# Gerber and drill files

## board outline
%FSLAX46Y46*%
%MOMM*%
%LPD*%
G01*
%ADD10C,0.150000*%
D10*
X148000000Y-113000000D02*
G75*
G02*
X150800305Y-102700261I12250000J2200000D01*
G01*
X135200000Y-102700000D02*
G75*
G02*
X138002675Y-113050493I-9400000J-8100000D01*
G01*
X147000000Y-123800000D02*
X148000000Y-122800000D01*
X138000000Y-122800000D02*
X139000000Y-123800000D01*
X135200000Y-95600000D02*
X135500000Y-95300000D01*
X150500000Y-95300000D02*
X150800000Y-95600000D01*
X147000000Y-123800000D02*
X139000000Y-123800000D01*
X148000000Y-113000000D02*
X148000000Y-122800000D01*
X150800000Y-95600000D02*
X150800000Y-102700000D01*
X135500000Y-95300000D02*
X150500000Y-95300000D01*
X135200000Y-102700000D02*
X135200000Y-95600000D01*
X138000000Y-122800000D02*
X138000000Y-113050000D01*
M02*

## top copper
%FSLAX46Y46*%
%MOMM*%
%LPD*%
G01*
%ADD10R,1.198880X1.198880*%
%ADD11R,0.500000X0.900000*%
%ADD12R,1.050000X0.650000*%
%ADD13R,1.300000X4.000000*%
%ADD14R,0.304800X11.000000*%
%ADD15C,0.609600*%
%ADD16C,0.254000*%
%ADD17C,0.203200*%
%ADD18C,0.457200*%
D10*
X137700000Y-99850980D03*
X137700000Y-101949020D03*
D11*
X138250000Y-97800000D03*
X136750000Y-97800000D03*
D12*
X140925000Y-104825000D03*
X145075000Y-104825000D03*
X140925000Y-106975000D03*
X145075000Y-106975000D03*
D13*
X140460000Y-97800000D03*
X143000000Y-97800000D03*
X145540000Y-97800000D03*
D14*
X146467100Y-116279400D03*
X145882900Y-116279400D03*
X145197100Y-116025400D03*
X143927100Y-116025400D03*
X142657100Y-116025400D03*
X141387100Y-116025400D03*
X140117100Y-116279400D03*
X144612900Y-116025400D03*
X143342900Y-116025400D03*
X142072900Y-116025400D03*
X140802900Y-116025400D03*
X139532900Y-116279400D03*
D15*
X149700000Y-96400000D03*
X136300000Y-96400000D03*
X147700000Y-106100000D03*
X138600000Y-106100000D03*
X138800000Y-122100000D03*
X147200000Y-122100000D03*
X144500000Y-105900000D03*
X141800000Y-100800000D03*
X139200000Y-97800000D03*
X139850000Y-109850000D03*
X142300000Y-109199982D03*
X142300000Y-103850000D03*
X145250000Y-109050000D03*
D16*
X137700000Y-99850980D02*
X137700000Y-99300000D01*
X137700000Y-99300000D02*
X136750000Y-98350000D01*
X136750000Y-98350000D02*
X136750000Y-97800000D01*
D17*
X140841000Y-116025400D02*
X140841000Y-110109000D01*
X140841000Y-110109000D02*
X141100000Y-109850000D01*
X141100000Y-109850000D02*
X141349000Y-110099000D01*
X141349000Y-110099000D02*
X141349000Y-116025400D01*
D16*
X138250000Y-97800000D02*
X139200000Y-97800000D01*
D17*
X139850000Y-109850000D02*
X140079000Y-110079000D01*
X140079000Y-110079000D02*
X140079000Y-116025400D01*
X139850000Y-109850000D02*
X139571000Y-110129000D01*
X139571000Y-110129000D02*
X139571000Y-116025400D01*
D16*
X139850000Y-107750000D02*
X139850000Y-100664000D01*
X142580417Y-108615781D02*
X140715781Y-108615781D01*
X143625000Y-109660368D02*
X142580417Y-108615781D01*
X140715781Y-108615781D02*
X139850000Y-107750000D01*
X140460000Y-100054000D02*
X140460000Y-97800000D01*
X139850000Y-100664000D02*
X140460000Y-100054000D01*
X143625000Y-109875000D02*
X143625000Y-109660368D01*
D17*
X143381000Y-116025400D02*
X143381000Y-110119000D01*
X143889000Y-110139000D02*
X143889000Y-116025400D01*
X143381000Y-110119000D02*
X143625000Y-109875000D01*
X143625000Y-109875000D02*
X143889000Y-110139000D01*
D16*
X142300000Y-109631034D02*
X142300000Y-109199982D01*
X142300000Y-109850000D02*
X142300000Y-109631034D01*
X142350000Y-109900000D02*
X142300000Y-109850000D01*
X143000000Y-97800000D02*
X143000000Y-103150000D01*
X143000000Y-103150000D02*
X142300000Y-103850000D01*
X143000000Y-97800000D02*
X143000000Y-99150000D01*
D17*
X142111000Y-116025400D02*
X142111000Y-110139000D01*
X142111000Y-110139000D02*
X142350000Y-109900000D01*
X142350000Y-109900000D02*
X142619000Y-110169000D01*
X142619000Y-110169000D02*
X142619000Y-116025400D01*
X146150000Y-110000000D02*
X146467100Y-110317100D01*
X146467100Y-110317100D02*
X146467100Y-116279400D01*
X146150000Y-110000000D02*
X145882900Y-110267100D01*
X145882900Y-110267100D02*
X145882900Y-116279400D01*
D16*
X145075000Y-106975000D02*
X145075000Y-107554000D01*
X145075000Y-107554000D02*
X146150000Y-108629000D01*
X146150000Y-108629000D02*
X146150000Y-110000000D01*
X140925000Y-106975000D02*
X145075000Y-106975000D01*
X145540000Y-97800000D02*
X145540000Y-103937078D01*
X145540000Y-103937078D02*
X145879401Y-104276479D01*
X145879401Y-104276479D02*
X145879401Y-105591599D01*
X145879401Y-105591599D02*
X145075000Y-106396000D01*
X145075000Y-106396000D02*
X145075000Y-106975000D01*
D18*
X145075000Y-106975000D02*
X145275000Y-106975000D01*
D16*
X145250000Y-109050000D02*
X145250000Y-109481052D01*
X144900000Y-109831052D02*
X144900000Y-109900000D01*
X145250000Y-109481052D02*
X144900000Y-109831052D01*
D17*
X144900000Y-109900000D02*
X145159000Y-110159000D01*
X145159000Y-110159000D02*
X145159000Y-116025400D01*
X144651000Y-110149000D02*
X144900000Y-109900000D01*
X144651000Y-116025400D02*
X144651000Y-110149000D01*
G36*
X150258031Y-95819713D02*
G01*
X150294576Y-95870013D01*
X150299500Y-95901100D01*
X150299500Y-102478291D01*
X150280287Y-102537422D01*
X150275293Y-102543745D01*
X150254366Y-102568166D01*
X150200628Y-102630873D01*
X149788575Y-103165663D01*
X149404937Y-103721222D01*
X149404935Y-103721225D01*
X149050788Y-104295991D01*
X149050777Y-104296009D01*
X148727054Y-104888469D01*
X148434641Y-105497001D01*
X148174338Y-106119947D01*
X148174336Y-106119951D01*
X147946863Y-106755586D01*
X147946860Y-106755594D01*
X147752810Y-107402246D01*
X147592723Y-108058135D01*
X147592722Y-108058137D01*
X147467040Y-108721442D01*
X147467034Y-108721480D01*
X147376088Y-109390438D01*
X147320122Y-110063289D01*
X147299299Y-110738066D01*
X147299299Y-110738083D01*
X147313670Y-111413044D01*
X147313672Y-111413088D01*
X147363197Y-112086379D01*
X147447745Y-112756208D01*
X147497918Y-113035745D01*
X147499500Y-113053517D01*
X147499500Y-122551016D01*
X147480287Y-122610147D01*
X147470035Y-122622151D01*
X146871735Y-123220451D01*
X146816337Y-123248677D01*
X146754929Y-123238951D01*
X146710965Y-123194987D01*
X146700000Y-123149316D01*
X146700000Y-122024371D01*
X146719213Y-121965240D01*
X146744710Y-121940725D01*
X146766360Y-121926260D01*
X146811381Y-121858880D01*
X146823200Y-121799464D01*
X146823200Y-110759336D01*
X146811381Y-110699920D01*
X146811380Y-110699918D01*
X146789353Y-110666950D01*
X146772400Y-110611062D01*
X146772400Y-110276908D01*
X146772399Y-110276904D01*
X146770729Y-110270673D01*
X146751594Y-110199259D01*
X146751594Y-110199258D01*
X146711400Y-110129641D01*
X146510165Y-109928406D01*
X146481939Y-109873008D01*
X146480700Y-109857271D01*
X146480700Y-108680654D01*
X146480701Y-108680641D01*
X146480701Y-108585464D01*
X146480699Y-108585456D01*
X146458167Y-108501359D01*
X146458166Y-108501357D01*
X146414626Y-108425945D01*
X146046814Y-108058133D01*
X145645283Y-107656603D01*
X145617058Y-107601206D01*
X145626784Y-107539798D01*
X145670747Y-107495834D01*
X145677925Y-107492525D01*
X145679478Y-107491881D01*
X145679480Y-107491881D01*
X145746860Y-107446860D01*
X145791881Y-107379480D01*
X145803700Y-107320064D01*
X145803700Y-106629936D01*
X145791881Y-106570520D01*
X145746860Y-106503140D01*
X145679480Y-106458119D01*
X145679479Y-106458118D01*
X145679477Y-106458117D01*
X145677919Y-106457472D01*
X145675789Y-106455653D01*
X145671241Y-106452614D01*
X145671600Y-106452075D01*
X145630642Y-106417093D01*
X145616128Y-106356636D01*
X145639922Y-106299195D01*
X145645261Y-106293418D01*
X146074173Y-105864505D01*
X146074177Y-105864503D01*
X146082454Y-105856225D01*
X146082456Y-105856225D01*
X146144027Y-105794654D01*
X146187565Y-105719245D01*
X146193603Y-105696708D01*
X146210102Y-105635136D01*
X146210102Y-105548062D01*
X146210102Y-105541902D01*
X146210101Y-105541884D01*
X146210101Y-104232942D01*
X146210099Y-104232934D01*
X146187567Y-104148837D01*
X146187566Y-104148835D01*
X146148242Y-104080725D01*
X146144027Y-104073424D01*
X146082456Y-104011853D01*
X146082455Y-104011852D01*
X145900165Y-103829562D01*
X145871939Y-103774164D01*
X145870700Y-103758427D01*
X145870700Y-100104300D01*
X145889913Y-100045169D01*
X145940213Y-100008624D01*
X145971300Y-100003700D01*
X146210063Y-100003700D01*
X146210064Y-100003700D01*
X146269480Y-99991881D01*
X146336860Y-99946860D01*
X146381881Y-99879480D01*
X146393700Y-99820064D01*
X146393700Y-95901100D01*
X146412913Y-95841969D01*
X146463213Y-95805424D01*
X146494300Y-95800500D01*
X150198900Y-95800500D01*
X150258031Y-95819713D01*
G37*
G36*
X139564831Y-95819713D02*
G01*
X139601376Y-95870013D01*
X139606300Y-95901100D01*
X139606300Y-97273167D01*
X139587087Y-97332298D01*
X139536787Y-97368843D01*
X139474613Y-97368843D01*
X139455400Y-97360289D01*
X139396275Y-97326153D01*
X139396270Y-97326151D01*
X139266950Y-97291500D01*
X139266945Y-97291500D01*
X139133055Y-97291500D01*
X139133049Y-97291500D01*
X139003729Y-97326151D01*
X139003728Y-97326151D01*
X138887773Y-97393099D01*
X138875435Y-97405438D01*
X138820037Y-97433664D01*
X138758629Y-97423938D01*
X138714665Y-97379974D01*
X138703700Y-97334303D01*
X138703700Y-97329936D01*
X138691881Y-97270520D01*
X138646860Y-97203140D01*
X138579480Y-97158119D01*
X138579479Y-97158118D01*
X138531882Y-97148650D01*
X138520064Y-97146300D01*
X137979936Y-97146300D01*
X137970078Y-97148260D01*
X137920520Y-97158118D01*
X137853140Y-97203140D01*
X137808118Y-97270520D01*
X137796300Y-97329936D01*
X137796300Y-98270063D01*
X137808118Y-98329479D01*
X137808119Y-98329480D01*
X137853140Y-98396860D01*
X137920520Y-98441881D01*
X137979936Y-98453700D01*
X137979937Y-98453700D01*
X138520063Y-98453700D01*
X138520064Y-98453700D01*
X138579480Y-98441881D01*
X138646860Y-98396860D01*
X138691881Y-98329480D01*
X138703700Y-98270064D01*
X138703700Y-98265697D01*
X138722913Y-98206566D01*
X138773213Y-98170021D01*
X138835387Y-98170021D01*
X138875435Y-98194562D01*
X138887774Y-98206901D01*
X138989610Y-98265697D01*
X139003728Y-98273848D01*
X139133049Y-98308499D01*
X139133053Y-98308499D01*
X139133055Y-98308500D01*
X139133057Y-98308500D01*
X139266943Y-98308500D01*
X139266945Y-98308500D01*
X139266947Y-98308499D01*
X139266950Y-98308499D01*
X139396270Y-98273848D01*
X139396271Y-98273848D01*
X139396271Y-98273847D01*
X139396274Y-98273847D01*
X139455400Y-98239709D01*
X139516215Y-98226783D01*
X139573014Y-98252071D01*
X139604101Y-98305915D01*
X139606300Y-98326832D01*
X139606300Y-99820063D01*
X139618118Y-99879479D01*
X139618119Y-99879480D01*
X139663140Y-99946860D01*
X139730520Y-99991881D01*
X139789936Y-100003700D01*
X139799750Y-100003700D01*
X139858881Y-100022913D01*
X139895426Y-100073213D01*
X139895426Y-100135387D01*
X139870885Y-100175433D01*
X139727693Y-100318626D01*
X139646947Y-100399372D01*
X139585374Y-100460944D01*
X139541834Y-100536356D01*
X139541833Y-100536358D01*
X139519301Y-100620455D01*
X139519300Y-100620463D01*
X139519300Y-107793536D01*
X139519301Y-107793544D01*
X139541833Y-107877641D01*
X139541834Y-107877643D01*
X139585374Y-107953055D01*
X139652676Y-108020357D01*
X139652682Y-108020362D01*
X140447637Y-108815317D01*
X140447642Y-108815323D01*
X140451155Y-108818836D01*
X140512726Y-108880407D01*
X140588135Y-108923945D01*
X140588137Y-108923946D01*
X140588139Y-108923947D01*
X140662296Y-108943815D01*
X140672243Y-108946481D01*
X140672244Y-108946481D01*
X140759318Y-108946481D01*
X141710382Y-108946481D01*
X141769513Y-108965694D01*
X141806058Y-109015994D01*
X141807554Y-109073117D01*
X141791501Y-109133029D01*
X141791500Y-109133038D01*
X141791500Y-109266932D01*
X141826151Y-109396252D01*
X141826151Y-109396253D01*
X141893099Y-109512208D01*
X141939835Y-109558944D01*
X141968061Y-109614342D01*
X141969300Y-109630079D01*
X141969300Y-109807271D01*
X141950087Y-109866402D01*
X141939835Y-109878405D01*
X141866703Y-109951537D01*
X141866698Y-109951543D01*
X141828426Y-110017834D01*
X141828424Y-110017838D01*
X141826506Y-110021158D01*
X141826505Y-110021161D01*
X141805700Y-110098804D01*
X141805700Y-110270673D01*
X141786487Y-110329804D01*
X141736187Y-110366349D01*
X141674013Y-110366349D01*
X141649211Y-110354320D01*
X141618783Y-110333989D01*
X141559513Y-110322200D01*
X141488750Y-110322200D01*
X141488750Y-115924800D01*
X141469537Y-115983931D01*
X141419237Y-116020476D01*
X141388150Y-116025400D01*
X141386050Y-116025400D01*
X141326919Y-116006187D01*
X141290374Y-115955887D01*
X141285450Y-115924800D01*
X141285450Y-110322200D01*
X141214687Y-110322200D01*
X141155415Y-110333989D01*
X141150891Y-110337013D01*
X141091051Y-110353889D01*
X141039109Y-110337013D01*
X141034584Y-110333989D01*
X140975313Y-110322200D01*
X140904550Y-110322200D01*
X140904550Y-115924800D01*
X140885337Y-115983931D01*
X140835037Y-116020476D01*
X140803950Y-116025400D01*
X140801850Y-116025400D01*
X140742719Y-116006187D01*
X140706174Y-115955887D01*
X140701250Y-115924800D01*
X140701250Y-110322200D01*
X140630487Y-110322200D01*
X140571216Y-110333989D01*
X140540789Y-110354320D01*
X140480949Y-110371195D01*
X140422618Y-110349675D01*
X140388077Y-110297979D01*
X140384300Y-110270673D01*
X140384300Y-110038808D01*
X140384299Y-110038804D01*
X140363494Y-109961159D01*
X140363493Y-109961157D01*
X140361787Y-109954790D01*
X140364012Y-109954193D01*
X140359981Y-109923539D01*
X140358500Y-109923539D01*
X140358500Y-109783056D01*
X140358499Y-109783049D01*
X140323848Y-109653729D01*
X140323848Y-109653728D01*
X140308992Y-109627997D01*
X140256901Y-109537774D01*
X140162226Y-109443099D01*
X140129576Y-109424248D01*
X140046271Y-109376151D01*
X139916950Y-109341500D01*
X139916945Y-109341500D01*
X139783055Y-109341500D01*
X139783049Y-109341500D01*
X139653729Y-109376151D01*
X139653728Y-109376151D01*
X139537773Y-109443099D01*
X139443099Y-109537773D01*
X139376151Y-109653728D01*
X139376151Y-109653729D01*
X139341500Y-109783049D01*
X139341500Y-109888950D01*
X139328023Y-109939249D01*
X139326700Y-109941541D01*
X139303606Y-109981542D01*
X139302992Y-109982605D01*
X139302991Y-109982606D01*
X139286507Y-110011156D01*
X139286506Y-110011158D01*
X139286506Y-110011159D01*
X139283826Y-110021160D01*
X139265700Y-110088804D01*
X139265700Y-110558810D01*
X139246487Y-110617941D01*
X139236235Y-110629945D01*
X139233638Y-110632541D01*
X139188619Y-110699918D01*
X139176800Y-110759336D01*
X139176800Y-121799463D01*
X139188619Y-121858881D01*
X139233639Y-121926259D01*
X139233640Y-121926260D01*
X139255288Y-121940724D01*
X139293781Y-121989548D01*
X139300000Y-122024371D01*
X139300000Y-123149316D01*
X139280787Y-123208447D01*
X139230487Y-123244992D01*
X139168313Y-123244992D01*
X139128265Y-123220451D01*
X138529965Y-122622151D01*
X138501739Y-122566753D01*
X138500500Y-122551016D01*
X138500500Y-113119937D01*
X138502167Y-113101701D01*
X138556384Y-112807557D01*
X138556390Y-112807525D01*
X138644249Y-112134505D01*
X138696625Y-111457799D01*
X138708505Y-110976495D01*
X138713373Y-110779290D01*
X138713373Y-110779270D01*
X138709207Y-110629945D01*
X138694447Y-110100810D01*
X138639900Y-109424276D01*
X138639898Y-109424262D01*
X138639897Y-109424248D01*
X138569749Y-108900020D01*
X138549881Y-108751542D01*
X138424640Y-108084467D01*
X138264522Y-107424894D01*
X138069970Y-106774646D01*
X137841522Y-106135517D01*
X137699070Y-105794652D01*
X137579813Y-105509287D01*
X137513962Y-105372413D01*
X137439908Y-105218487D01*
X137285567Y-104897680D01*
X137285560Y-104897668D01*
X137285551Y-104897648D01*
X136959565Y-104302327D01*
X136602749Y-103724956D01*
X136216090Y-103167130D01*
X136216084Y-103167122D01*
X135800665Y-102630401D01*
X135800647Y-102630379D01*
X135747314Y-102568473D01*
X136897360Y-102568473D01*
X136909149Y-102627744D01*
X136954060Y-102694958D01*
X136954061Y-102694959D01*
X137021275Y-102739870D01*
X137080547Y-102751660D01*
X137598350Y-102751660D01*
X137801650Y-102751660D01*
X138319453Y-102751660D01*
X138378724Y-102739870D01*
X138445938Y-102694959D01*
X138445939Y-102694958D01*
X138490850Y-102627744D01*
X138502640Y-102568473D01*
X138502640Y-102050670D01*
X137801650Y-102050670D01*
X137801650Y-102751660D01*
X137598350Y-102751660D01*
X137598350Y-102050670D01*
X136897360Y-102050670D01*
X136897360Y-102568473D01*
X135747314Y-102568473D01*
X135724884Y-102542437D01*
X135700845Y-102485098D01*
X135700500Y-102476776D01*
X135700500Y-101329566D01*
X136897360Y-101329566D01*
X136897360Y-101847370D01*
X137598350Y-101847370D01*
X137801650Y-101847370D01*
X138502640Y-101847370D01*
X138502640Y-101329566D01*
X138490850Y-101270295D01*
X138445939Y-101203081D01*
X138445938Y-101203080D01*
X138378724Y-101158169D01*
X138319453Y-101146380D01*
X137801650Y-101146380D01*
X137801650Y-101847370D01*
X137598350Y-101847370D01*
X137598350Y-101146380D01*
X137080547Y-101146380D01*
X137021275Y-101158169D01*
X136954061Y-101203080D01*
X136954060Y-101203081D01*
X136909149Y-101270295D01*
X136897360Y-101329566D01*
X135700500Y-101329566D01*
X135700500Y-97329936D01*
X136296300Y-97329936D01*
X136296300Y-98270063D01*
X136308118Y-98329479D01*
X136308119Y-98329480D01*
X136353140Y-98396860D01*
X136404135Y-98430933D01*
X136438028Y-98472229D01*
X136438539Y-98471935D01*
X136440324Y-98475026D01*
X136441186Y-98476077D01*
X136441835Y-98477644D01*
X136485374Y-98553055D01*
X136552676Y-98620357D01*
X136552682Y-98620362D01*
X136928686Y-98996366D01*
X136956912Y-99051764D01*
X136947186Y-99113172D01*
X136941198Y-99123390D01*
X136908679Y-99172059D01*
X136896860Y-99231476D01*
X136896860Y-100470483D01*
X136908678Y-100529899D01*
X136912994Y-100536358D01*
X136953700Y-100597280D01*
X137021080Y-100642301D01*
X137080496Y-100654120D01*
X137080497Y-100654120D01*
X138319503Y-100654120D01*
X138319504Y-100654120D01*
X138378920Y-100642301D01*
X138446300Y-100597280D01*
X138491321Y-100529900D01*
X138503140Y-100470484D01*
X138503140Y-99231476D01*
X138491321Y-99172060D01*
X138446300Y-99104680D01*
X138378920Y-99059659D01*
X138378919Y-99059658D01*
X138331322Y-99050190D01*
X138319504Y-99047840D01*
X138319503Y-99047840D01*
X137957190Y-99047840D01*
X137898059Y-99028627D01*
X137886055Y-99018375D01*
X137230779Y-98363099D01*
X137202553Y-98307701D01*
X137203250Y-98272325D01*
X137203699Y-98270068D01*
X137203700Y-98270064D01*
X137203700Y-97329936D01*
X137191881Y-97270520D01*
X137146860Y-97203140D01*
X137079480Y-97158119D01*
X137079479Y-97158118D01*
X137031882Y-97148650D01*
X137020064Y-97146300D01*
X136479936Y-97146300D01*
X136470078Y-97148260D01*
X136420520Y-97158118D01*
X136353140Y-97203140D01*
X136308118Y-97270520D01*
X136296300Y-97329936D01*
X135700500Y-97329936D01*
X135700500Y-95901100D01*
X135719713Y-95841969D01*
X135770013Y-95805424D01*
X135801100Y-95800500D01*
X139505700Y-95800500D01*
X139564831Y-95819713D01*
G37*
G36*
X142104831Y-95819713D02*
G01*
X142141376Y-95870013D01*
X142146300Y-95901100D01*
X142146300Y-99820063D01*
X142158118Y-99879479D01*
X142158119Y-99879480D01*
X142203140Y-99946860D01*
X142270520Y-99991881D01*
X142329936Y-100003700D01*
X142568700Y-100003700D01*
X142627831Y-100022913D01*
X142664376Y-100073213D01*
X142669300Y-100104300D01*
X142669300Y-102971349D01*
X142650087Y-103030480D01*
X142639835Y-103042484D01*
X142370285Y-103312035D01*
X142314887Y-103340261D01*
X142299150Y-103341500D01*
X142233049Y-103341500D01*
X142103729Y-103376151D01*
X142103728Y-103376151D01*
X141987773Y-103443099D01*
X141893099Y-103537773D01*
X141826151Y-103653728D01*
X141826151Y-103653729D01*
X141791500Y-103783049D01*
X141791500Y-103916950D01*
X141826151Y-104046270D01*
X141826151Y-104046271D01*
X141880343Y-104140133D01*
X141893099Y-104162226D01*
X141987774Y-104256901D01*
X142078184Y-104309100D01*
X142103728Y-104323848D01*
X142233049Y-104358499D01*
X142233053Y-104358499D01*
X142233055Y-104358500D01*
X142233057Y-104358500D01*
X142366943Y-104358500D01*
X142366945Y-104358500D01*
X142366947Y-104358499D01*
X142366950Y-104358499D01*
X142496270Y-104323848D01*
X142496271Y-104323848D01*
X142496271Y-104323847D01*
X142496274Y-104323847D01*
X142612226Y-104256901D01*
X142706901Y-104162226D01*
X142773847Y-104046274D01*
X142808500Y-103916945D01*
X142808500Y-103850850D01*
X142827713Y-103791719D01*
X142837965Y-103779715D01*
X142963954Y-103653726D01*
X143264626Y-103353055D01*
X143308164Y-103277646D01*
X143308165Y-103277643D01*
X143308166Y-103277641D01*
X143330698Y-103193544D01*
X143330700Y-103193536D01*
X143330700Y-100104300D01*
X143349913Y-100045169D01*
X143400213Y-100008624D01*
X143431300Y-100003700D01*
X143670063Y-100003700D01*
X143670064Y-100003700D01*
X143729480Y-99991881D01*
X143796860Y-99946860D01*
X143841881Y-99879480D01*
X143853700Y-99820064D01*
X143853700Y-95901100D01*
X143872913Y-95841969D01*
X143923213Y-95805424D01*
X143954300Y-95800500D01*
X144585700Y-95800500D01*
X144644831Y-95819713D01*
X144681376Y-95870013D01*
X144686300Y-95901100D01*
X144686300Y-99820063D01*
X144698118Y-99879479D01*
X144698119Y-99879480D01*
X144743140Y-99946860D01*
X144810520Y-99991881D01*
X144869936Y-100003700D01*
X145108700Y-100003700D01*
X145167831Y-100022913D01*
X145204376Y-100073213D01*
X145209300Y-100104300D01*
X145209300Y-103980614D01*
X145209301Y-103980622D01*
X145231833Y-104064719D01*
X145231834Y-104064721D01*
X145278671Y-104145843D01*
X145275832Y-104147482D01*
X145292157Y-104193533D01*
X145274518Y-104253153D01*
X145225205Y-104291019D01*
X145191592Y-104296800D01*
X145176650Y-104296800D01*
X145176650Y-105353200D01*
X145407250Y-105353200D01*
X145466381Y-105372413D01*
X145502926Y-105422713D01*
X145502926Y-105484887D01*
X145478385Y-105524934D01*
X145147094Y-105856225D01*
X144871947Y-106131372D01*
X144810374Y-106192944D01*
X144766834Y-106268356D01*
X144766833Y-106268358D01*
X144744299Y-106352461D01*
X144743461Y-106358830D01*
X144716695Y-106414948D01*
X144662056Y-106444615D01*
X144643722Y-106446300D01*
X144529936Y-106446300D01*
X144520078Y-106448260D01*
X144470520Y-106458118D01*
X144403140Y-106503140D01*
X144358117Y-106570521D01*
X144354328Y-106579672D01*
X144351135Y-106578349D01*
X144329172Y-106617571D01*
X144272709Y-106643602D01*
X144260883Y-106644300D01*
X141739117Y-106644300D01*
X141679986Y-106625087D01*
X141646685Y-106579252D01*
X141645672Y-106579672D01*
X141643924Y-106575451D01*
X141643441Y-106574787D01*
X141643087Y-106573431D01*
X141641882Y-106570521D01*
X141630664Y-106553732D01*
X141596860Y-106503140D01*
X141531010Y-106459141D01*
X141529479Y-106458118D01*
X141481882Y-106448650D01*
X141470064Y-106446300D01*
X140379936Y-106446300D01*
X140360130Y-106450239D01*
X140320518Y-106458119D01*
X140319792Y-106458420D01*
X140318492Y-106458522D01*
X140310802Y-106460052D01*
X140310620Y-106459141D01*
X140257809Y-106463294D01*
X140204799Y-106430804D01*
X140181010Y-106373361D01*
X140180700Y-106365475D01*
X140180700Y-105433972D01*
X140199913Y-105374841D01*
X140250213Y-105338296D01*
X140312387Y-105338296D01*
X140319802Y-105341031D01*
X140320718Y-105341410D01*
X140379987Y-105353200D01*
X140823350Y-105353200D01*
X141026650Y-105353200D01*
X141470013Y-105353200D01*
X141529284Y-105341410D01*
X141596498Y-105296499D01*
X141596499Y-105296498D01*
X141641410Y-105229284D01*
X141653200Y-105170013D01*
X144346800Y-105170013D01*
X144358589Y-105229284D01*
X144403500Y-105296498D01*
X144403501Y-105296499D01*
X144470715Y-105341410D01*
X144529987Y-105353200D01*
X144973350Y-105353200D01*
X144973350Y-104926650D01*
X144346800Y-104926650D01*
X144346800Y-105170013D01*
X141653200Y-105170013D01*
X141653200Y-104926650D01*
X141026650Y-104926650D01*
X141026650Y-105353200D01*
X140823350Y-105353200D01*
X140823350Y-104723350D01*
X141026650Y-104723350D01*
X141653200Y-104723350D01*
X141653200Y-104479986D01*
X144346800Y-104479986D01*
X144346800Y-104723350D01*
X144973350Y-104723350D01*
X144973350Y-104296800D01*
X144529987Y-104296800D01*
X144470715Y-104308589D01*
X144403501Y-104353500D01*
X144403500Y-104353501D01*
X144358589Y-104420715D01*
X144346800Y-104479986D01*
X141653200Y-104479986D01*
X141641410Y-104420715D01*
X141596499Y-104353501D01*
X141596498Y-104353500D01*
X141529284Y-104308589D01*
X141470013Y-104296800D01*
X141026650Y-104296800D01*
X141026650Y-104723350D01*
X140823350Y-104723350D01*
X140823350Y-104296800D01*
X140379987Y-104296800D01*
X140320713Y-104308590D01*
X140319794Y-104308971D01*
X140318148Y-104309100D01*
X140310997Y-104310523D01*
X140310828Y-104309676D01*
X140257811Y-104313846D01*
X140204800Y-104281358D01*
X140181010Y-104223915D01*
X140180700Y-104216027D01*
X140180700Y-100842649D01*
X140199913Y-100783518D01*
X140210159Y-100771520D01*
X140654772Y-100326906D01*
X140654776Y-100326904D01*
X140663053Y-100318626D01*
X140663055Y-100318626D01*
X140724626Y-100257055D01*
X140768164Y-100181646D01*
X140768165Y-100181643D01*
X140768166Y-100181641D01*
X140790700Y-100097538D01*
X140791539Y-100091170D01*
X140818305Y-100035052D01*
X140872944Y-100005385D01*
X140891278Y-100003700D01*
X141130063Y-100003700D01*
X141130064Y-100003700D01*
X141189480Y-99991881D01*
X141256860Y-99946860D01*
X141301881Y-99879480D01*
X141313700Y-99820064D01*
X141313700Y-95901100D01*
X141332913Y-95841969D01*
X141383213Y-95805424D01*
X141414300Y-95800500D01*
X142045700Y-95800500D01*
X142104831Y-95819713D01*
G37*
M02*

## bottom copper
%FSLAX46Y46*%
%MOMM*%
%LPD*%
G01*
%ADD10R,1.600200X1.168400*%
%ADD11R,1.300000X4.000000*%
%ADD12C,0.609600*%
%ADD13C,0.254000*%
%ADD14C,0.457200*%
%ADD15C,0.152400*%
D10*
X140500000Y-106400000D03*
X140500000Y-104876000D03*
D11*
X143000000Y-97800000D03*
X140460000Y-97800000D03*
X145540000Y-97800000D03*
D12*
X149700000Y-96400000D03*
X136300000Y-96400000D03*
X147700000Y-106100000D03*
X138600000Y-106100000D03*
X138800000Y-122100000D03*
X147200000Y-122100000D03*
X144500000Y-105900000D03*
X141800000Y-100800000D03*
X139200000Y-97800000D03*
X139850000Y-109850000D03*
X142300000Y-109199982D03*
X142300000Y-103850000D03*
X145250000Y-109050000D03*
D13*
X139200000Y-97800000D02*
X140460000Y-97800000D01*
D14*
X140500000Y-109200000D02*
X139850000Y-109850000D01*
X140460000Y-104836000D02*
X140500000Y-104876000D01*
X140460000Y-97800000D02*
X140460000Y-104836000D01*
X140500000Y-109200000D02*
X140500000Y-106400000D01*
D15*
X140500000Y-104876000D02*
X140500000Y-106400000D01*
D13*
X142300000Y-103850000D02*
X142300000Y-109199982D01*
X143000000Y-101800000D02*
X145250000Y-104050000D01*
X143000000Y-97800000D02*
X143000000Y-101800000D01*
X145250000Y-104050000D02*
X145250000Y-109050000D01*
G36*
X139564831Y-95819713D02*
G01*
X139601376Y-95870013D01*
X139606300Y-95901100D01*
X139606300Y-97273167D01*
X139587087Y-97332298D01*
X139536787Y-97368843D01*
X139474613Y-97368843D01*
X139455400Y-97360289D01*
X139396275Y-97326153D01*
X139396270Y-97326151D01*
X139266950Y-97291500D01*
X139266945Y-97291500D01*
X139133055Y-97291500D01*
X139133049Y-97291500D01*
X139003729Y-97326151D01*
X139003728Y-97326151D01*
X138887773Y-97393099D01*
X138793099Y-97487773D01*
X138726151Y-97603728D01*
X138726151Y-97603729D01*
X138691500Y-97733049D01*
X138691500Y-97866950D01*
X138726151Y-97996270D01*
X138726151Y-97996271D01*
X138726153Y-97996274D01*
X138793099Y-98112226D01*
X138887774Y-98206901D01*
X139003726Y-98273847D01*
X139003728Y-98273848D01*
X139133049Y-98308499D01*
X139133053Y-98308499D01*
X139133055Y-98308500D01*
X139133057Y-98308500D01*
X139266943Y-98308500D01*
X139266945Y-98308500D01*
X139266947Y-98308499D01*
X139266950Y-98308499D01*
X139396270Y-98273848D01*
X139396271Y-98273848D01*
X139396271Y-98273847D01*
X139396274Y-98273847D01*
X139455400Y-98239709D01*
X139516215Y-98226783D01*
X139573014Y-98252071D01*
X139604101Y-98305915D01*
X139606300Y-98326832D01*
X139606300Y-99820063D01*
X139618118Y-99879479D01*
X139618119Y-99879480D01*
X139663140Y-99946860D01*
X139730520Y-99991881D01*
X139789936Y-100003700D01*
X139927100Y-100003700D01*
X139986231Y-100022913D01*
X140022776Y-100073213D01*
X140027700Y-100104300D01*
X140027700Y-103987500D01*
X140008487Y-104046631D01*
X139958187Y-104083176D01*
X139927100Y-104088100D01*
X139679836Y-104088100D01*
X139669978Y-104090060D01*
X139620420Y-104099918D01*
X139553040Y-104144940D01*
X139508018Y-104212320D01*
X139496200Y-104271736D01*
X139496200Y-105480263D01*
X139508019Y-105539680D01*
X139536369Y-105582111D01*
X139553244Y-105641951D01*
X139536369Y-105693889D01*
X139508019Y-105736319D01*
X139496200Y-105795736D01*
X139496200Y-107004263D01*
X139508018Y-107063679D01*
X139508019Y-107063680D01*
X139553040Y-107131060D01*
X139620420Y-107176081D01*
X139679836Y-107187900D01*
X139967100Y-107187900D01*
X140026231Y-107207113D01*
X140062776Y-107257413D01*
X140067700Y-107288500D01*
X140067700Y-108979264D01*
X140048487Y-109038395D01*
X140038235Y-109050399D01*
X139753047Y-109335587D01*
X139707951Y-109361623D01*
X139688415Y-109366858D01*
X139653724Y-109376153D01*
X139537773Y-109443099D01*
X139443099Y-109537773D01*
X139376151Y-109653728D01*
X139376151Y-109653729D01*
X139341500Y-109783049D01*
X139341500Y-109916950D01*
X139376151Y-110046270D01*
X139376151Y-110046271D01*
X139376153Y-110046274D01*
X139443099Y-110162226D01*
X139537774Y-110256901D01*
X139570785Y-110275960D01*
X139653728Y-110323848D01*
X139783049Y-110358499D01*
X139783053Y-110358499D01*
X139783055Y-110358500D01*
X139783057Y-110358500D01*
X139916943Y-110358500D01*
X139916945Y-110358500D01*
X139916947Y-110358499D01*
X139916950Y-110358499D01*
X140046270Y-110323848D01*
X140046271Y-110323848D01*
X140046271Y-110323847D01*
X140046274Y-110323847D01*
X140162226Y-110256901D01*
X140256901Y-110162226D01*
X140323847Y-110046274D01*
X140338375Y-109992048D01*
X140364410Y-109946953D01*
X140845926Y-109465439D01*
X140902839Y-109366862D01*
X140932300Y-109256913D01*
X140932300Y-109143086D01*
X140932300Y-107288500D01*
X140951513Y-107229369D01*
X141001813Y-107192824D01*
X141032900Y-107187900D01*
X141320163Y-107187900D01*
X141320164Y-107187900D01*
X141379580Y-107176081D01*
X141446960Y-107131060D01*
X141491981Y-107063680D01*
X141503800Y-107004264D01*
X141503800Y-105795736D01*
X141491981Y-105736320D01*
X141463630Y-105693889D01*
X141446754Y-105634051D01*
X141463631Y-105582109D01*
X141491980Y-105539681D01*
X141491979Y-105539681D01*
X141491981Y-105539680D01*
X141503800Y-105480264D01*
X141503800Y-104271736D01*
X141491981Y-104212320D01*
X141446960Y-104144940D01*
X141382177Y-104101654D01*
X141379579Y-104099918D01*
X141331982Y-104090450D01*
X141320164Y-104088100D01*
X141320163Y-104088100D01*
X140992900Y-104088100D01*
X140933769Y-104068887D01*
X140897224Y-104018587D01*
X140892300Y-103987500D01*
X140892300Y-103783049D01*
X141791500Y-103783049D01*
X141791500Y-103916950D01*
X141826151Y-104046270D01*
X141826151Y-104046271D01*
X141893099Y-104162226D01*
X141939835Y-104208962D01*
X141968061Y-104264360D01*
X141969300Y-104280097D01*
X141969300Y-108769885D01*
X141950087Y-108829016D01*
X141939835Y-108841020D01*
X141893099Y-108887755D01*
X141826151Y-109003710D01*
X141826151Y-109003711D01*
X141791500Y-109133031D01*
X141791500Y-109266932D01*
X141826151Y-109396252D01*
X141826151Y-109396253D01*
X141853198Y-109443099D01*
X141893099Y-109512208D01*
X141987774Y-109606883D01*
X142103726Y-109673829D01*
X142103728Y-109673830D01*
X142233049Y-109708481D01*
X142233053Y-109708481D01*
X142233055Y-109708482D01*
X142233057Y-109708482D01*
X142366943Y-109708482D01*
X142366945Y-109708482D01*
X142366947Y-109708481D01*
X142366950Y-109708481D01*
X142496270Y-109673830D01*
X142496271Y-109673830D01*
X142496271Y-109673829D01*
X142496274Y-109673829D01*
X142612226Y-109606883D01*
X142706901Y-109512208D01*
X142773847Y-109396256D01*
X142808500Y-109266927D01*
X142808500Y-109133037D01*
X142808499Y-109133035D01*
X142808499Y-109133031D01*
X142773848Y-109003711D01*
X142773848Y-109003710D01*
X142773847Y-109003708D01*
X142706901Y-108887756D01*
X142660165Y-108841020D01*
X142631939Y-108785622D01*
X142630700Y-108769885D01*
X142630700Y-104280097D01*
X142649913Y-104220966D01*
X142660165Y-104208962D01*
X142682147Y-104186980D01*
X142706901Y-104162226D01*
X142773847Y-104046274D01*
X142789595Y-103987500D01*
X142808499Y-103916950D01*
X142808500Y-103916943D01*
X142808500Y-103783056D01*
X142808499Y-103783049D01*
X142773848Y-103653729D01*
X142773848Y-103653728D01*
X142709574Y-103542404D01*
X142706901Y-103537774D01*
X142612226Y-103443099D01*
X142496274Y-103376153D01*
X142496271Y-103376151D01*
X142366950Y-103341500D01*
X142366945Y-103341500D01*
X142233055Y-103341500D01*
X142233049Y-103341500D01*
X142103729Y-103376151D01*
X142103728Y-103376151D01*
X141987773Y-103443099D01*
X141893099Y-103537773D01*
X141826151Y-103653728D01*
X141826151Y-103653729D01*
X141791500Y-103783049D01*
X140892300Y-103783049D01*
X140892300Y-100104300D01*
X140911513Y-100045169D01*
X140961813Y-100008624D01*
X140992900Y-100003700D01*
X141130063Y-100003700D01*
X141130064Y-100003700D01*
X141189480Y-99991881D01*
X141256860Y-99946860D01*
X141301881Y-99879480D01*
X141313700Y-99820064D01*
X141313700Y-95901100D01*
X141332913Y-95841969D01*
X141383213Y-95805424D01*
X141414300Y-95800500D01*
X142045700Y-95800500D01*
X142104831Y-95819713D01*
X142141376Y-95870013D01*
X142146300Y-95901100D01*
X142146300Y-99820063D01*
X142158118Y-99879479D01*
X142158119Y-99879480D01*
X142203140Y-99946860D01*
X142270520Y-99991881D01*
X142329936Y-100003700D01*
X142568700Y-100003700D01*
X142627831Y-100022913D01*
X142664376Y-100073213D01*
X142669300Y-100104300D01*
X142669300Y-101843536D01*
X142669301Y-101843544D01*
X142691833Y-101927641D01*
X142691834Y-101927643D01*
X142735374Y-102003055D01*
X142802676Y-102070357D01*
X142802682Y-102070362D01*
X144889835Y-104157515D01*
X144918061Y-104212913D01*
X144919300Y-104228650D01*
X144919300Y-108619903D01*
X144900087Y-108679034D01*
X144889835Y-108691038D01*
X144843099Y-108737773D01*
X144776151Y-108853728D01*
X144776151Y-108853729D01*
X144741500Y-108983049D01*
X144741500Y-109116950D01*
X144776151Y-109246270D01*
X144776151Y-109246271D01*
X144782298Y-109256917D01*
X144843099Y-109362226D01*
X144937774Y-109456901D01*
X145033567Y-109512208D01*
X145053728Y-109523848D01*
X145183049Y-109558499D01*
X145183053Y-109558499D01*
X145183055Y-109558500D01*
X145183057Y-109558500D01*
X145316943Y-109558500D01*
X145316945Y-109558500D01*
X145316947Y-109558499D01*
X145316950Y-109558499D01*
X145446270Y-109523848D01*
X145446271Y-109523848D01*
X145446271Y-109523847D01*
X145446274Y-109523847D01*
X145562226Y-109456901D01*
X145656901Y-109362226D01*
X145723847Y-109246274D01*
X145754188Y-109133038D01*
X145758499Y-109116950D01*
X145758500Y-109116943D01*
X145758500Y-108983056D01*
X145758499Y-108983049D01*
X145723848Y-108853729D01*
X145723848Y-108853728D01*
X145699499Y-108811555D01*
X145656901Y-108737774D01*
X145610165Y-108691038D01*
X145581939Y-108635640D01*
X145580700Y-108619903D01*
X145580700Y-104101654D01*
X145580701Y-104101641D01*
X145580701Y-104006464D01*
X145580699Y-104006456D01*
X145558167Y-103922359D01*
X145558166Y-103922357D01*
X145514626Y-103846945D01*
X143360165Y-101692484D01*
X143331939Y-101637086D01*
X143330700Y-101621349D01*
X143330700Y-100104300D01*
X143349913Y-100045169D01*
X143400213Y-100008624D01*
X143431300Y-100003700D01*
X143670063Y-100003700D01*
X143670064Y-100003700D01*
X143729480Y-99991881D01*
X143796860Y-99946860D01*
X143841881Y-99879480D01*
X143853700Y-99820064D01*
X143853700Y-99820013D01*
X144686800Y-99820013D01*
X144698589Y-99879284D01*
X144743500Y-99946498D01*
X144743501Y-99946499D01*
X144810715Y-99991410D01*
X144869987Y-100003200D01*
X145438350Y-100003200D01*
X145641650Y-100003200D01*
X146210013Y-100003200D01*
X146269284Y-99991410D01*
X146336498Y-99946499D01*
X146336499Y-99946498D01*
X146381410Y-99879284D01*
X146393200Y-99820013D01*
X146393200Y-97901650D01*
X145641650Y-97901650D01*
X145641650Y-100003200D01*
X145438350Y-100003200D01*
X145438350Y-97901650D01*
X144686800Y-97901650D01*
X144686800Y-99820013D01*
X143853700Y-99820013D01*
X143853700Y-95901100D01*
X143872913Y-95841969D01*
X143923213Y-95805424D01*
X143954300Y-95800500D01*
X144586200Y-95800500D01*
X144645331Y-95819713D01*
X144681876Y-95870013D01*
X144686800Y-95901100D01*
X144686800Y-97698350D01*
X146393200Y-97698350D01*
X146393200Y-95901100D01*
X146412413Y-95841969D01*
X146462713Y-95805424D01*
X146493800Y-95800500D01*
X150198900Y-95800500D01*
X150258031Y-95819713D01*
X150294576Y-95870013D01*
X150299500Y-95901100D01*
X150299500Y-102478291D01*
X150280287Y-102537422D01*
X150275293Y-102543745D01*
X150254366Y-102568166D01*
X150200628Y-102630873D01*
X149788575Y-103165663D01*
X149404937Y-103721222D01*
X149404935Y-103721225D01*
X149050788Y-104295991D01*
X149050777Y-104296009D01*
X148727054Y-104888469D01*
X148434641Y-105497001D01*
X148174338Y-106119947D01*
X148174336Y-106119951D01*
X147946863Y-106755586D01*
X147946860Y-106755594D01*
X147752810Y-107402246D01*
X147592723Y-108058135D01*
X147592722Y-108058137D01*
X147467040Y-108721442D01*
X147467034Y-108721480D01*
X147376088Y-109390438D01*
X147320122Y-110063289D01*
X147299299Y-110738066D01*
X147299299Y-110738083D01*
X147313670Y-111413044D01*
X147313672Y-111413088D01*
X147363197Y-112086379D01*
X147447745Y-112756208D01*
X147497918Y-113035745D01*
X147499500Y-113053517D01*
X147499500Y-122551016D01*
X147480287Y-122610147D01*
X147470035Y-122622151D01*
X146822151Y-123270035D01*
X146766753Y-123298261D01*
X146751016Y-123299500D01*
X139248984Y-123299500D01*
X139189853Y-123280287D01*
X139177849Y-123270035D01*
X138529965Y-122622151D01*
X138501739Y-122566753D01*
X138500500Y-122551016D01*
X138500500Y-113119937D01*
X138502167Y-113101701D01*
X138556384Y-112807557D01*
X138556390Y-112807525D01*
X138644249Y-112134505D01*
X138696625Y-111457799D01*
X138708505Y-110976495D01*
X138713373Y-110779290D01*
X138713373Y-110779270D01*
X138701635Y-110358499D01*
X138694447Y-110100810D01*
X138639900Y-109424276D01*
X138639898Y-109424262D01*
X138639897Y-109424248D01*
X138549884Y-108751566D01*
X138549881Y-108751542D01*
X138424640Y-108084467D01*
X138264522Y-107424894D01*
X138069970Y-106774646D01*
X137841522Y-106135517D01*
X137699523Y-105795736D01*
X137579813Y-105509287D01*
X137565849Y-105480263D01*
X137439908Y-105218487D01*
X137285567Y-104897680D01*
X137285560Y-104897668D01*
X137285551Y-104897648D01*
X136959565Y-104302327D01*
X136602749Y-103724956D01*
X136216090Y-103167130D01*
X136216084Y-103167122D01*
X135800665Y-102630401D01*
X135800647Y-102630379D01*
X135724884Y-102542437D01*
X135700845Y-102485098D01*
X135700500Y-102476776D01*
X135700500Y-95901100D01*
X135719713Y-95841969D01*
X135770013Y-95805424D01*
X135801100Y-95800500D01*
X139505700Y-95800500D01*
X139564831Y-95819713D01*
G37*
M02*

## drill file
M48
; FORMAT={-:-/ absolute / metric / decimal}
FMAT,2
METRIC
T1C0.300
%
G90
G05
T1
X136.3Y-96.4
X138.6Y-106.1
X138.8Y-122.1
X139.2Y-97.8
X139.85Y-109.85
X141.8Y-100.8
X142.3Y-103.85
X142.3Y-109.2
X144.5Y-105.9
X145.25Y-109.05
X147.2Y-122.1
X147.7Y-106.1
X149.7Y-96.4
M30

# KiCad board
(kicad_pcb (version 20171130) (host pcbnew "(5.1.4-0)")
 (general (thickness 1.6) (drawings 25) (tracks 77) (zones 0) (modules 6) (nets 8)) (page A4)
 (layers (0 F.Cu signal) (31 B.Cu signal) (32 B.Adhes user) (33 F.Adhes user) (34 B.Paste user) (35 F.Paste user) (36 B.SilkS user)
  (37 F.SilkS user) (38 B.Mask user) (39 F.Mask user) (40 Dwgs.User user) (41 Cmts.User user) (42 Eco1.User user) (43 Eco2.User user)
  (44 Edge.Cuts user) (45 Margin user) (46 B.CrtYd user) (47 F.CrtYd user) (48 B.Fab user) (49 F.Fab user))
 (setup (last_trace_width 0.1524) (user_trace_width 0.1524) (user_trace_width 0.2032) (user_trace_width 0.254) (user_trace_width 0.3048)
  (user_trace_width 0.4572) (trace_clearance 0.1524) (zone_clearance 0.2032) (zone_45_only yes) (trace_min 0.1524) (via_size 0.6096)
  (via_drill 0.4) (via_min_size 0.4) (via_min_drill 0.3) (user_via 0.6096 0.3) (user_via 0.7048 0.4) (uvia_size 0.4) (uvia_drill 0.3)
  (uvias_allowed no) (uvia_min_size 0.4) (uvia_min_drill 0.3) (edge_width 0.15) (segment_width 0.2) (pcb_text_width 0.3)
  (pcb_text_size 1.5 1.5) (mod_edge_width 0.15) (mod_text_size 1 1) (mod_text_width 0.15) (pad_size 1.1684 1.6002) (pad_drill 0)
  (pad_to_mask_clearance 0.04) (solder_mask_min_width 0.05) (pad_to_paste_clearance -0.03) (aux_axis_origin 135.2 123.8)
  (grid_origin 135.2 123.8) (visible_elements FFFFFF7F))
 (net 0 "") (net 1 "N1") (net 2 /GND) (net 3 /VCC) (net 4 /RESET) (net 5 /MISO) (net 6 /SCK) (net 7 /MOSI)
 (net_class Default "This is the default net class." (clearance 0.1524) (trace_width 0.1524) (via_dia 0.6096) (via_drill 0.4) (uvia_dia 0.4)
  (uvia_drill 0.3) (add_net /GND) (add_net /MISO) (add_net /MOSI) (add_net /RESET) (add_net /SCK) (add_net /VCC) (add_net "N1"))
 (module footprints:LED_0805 (layer F.Cu) (at 137.7 100.9 90)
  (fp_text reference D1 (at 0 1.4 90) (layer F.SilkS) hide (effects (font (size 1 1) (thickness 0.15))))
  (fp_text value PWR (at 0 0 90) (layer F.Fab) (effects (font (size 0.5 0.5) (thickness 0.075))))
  (pad 2 smd rect (at 1.04902 0 270) (size 1.19888 1.19888) (layers F.Cu F.Paste F.Mask) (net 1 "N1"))
  (pad 1 smd rect (at -1.04902 0 270) (size 1.19888 1.19888) (layers F.Cu F.Paste F.Mask) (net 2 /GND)))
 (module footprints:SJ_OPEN (layer B.Cu) (at 140.5 105.638 90)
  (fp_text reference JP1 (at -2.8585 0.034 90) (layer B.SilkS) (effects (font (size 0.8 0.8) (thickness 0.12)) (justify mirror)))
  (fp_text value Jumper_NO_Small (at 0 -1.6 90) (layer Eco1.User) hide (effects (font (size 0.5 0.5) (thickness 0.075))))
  (pad 1 smd rect (at -0.762 0 90) (size 1.1684 1.6002) (layers B.Cu B.Mask) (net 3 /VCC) (solder_mask_margin 0.18))
  (pad 2 smd rect (at 0.762 0 90) (size 1.1684 1.6002) (layers B.Cu B.Mask) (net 3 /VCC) (solder_mask_margin 0.18)))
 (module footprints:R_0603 (layer F.Cu) (at 137.5 97.8 180)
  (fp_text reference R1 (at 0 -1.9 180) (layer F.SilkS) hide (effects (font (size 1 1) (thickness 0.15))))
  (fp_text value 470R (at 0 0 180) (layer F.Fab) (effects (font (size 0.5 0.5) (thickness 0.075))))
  (pad 1 smd rect (at -0.75 0 180) (size 0.5 0.9) (layers F.Cu F.Paste F.Mask) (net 3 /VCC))
  (pad 2 smd rect (at 0.75 0 180) (size 0.5 0.9) (layers F.Cu F.Paste F.Mask) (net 1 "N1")))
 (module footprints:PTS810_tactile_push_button (layer F.Cu) (at 143 105.9 270)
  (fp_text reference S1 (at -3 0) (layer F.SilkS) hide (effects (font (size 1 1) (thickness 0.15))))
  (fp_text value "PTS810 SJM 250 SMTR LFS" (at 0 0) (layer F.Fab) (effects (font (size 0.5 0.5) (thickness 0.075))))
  (pad 1 smd rect (at -1.075 2.075) (size 1.05 0.65) (layers F.Cu F.Paste F.Mask) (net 2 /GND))
  (pad 1 smd rect (at -1.075 -2.075) (size 1.05 0.65) (layers F.Cu F.Paste F.Mask) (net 2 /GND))
  (pad 2 smd rect (at 1.075 2.075) (size 1.05 0.65) (layers F.Cu F.Paste F.Mask) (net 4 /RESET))
  (pad 2 smd rect (at 1.075 -2.075) (size 1.05 0.65) (layers F.Cu F.Paste F.Mask) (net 4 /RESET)))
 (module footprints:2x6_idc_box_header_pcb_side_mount (layer F.Cu) (at 143 97.8)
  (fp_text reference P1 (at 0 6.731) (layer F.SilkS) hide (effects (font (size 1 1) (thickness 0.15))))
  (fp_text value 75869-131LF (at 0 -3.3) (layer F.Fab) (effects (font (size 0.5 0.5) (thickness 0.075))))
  (pad 1 smd rect (at -2.54 0) (size 1.3 4) (layers F.Cu F.Mask) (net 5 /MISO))
  (pad 3 smd rect (at 0 0) (size 1.3 4) (layers F.Cu F.Mask) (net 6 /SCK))
  (pad 5 smd rect (at 2.54 0) (size 1.3 4) (layers F.Cu F.Mask) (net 4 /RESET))
  (pad 4 smd rect (at 0 0) (size 1.3 4) (layers B.Cu B.Mask) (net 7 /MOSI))
  (pad 2 smd rect (at -2.54 0) (size 1.3 4) (layers B.Cu B.Mask) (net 3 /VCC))
  (pad 6 smd rect (at 2.54 0) (size 1.3 4) (layers B.Cu B.Mask) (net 2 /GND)))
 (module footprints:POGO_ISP (layer F.Cu) (at 143 116 180)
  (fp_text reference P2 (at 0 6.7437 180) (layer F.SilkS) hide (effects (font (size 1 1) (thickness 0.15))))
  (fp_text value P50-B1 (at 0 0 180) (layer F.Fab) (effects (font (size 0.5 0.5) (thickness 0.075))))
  (pad 5 smd rect (at -3.4671 -0.2794 180) (size 0.3048 11) (layers F.Cu F.Mask) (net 4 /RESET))
  (pad 5 smd rect (at -2.8829 -0.2794 180) (size 0.3048 11) (layers F.Cu F.Mask) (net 4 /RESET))
  (pad "" smd rect (at -3.4671 -4.7752 180) (size 0.3048 2) (layers F.Paste))
  (pad 12 smd rect (at -3.4671 -1.7752 180) (size 0.3048 2) (layers F.Paste))
  (pad 13 smd rect (at -3.4671 1.2248 180) (size 0.3048 2) (layers F.Paste))
  (pad "" smd rect (at -3.4671 4.2248 180) (size 0.3048 2) (layers F.Paste))
  (pad "" smd rect (at -2.8829 -4.7752 180) (size 0.3048 2) (layers F.Paste))
  (pad 12 smd rect (at -2.8829 -1.7752 180) (size 0.3048 2) (layers F.Paste))
  (pad 13 smd rect (at -2.8829 1.2248 180) (size 0.3048 2) (layers F.Paste))
  (pad "" smd rect (at -2.8829 4.2248 180) (size 0.3048 2) (layers F.Paste))
  (pad 4 smd rect (at -2.1971 -0.0254 180) (size 0.3048 11) (layers F.Cu F.Mask) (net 7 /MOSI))
  (pad 1 smd rect (at -0.9271 -0.0254 180) (size 0.3048 11) (layers F.Cu F.Mask) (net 5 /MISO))
  (pad 3 smd rect (at 0.3429 -0.0254 180) (size 0.3048 11) (layers F.Cu F.Mask) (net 6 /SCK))
  (pad 6 smd rect (at 1.6129 -0.0254 180) (size 0.3048 11) (layers F.Cu F.Mask) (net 2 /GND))
  (pad 2 smd rect (at 2.8829 -0.2794 180) (size 0.3048 11) (layers F.Cu F.Mask) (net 3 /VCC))
  (pad 4 smd rect (at -1.6129 -0.0254 180) (size 0.3048 11) (layers F.Cu F.Mask) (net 7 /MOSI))
  (pad 1 smd rect (at -0.3429 -0.0254 180) (size 0.3048 11) (layers F.Cu F.Mask) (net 5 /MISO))
  (pad 3 smd rect (at 0.9271 -0.0254 180) (size 0.3048 11) (layers F.Cu F.Mask) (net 6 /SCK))
  (pad 6 smd rect (at 2.1971 -0.0254 180) (size 0.3048 11) (layers F.Cu F.Mask) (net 2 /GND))
  (pad 2 smd rect (at 3.4671 -0.2794 180) (size 0.3048 11) (layers F.Cu F.Mask) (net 3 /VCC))
  (pad "" smd rect (at -2.1971 -4.5212 180) (size 0.3048 2) (layers F.Paste))
  (pad "" smd rect (at -0.9271 -4.5212 180) (size 0.3048 2) (layers F.Paste))
  (pad 61 smd rect (at 2.8829 -4.7752 180) (size 0.3048 2) (layers F.Paste))
  (pad 21 smd rect (at -2.1971 1.4788 180) (size 0.3048 2) (layers F.Paste))
  (pad 31 smd rect (at -0.9271 1.4788 180) (size 0.3048 2) (layers F.Paste))
  (pad 41 smd rect (at 0.3429 1.4788 180) (size 0.3048 2) (layers F.Paste))
  (pad 51 smd rect (at 1.6129 1.4788 180) (size 0.3048 2) (layers F.Paste))
  (pad 61 smd rect (at 2.8829 1.2248 180) (size 0.3048 2) (layers F.Paste))
  (pad 21 smd rect (at -2.1971 -1.5212 180) (size 0.3048 2) (layers F.Paste))
  (pad 31 smd rect (at -0.9271 -1.5212 180) (size 0.3048 2) (layers F.Paste))
  (pad 41 smd rect (at 0.3429 -1.5212 180) (size 0.3048 2) (layers F.Paste))
  (pad 51 smd rect (at 1.6129 -1.5212 180) (size 0.3048 2) (layers F.Paste))
  (pad 61 smd rect (at 2.8829 -1.7752 180) (size 0.3048 2) (layers F.Paste))
  (pad 21 smd rect (at -2.1971 4.4788 180) (size 0.3048 2) (layers F.Paste))
  (pad 31 smd rect (at -0.9271 4.4788 180) (size 0.3048 2) (layers F.Paste))
  (pad 41 smd rect (at 0.3429 4.4788 180) (size 0.3048 2) (layers F.Paste))
  (pad 51 smd rect (at 1.6129 4.4788 180) (size 0.3048 2) (layers F.Paste))
  (pad 61 smd rect (at 2.8829 4.2248 180) (size 0.3048 2) (layers F.Paste))
  (pad 21 smd rect (at -1.6129 4.4788 180) (size 0.3048 2) (layers F.Paste))
  (pad 31 smd rect (at -0.3429 4.4788 180) (size 0.3048 2) (layers F.Paste))
  (pad 41 smd rect (at 0.9271 4.4788 180) (size 0.3048 2) (layers F.Paste))
  (pad 51 smd rect (at 2.1971 4.4788 180) (size 0.3048 2) (layers F.Paste))
  (pad 61 smd rect (at 3.4671 4.2248 180) (size 0.3048 2) (layers F.Paste))
  (pad 21 smd rect (at -1.6129 1.4788 180) (size 0.3048 2) (layers F.Paste))
  (pad 31 smd rect (at -0.3429 1.4788 180) (size 0.3048 2) (layers F.Paste))
  (pad 41 smd rect (at 0.9271 1.4788 180) (size 0.3048 2) (layers F.Paste))
  (pad 51 smd rect (at 2.1971 1.4788 180) (size 0.3048 2) (layers F.Paste))
  (pad 61 smd rect (at 3.4671 1.2248 180) (size 0.3048 2) (layers F.Paste))
  (pad 21 smd rect (at -1.6129 -1.5212 180) (size 0.3048 2) (layers F.Paste))
  (pad 31 smd rect (at -0.3429 -1.5212 180) (size 0.3048 2) (layers F.Paste))
  (pad 41 smd rect (at 0.9271 -1.5212 180) (size 0.3048 2) (layers F.Paste))
  (pad 51 smd rect (at 2.1971 -1.5212 180) (size 0.3048 2) (layers F.Paste))
  (pad 61 smd rect (at 3.4671 -1.7752 180) (size 0.3048 2) (layers F.Paste))
  (pad "" smd rect (at -1.6129 -4.5212 180) (size 0.3048 2) (layers F.Paste))
  (pad "" smd rect (at -0.3429 -4.5212 180) (size 0.3048 2) (layers F.Paste))
  (pad 61 smd rect (at 3.4671 -4.7752 180) (size 0.3048 2) (layers F.Paste))
  (pad 0 smd rect (at 0.3429 -4.5212 180) (size 0.3048 2) (layers F.Paste))
  (pad 31 smd rect (at 1.6129 -4.5212 180) (size 0.3048 2) (layers F.Paste))
  (pad "" smd rect (at 0.9271 -4.5212 180) (size 0.3048 2) (layers F.Paste))
  (pad 31 smd rect (at 2.1971 -4.5212 180) (size 0.3048 2) (layers F.Paste))
  (pad "" smd rect (at -3.175 -0.2794 180) (size 0.3048 11) (layers F.Mask))
  (pad "" smd rect (at -1.905 -0.0254 180) (size 0.3048 11) (layers F.Mask))
  (pad "" smd rect (at -0.635 -0.0254 180) (size 0.3048 11) (layers F.Mask))
  (pad "" smd rect (at 0.635 -0.0254 180) (size 0.3048 11) (layers F.Mask))
  (pad "" smd rect (at 1.905 -0.0254 180) (size 0.3048 11) (layers F.Mask))
  (pad "" smd rect (at 3.175 -0.2794 180) (size 0.3048 11) (layers F.Mask)))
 (gr_arc (start 160.25 110.8) (end 148 113) (angle 50.78261565) (layer Edge.Cuts) (width 0.15))
 (gr_arc (start 125.8 110.8) (end 135.2 102.7) (angle 51.20097292) (layer Edge.Cuts) (width 0.15))
 (gr_line (start 147 123.8) (end 148 122.8) (layer Edge.Cuts) (width 0.15))
 (gr_line (start 138 122.8) (end 139 123.8) (layer Edge.Cuts) (width 0.15))
 (gr_line (start 135.2 95.6) (end 135.5 95.3) (layer Edge.Cuts) (width 0.15))
 (gr_line (start 150.5 95.3) (end 150.8 95.6) (layer Edge.Cuts) (width 0.15))
 (gr_line (start 147 123.8) (end 139 123.8) (layer Edge.Cuts) (width 0.15))
 (gr_line (start 148 113) (end 148 122.8) (layer Edge.Cuts) (width 0.15))
 (gr_line (start 150.8 95.6) (end 150.8 102.7) (layer Edge.Cuts) (width 0.15))
 (gr_line (start 135.5 95.3) (end 150.5 95.3) (layer Edge.Cuts) (width 0.15))
 (gr_line (start 135.2 102.7) (end 135.2 95.6) (layer Edge.Cuts) (width 0.15))
 (gr_line (start 138 122.8) (end 138 113.05) (layer Edge.Cuts) (width 0.15))
 (segment (start 137.7 99.85098) (end 137.7 99.3) (width 0.254) (layer F.Cu) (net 1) (status 30))
 (segment (start 137.7 99.3) (end 136.75 98.35) (width 0.254) (layer F.Cu) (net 1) (status 10))
 (segment (start 136.75 98.35) (end 136.75 97.8) (width 0.254) (layer F.Cu) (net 1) (status 20))
 (segment (start 140.841 116.0254) (end 140.841 110.109) (width 0.2032) (layer F.Cu) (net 2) (status 10))
 (segment (start 140.841 110.109) (end 141.1 109.85) (width 0.2032) (layer F.Cu) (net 2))
 (segment (start 141.1 109.85) (end 141.349 110.099) (width 0.2032) (layer F.Cu) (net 2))
 (segment (start 141.349 110.099) (end 141.349 116.0254) (width 0.2032) (layer F.Cu) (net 2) (status 20))
 (via (at 149.7 96.4) (size 0.6096) (drill 0.3) (layers F.Cu B.Cu) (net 2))
 (via (at 136.3 96.4) (size 0.6096) (drill 0.3) (layers F.Cu B.Cu) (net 2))
 (via (at 147.7 106.1) (size 0.6096) (drill 0.3) (layers F.Cu B.Cu) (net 2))
 (via (at 138.6 106.1) (size 0.6096) (drill 0.3) (layers F.Cu B.Cu) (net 2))
 (via (at 138.8 122.1) (size 0.6096) (drill 0.3) (layers F.Cu B.Cu) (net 2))
 (via (at 147.2 122.1) (size 0.6096) (drill 0.3) (layers F.Cu B.Cu) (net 2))
 (via (at 144.5 105.9) (size 0.6096) (drill 0.3) (layers F.Cu B.Cu) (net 2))
 (via (at 141.8 100.8) (size 0.6096) (drill 0.3) (layers F.Cu B.Cu) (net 2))
 (segment (start 139.2 97.8) (end 140.46 97.8) (width 0.254) (layer B.Cu) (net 3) (status 20))
 (segment (start 138.25 97.8) (end 139.2 97.8) (width 0.254) (layer F.Cu) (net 3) (status 10))
 (via (at 139.2 97.8) (size 0.6096) (drill 0.3) (layers F.Cu B.Cu) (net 3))
 (segment (start 139.85 109.85) (end 140.079 110.079) (width 0.2032) (layer F.Cu) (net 3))
 (segment (start 140.079 110.079) (end 140.079 116.0254) (width 0.2032) (layer F.Cu) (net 3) (status 20))
 (segment (start 139.85 109.85) (end 139.571 110.129) (width 0.2032) (layer F.Cu) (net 3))
 (segment (start 139.571 110.129) (end 139.571 116.0254) (width 0.2032) (layer F.Cu) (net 3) (status 20))
 (via (at 139.85 109.85) (size 0.6096) (drill 0.3) (layers F.Cu B.Cu) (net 3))
 (segment (start 140.5 109.2) (end 139.85 109.85) (width 0.4572) (layer B.Cu) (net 3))
 (segment (start 140.46 104.836) (end 140.5 104.876) (width 0.4572) (layer B.Cu) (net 3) (status 30))
 (segment (start 140.46 97.8) (end 140.46 104.836) (width 0.4572) (layer B.Cu) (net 3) (status 30))
 (segment (start 140.5 109.2) (end 140.5 106.4) (width 0.4572) (layer B.Cu) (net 3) (status 20))
 (segment (start 140.5 104.876) (end 140.5 106.4) (width 0.1524) (layer B.Cu) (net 3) (status 30))
 (segment (start 139.85 107.75) (end 139.85 100.664) (width 0.254) (layer F.Cu) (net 5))
 (segment (start 142.580417 108.615781) (end 140.715781 108.615781) (width 0.254) (layer F.Cu) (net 5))
 (segment (start 143.625 109.660368) (end 142.580417 108.615781) (width 0.254) (layer F.Cu) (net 5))
 (segment (start 140.715781 108.615781) (end 139.85 107.75) (width 0.254) (layer F.Cu) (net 5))
 (segment (start 140.46 100.054) (end 140.46 97.8) (width 0.254) (layer F.Cu) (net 5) (status 20))
 (segment (start 139.85 100.664) (end 140.46 100.054) (width 0.254) (layer F.Cu) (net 5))
 (segment (start 143.625 109.875) (end 143.625 109.660368) (width 0.254) (layer F.Cu) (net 5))
 (segment (start 143.381 116.0254) (end 143.381 110.119) (width 0.2032) (layer F.Cu) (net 5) (status 10))
 (segment (start 143.889 110.139) (end 143.889 116.0254) (width 0.2032) (layer F.Cu) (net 5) (status 20))
 (segment (start 143.381 110.119) (end 143.625 109.875) (width 0.2032) (layer F.Cu) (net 5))
 (segment (start 143.625 109.875) (end 143.889 110.139) (width 0.2032) (layer F.Cu) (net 5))
 (segment (start 142.3 109.631034) (end 142.3 109.199982) (width 0.254) (layer F.Cu) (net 6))
 (segment (start 142.3 109.85) (end 142.3 109.631034) (width 0.254) (layer F.Cu) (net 6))
 (segment (start 142.35 109.9) (end 142.3 109.85) (width 0.254) (layer F.Cu) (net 6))
 (segment (start 142.3 103.85) (end 142.3 109.199982) (width 0.254) (layer B.Cu) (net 6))
 (via (at 142.3 109.199982) (size 0.6096) (drill 0.3) (layers F.Cu B.Cu) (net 6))
 (segment (start 143 97.8) (end 143 103.15) (width 0.254) (layer F.Cu) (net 6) (status 10))
 (segment (start 143 103.15) (end 142.3 103.85) (width 0.254) (layer F.Cu) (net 6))
 (via (at 142.3 103.85) (size 0.6096) (drill 0.3) (layers F.Cu B.Cu) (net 6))
 (segment (start 143 97.8) (end 143 99.15) (width 0.254) (layer F.Cu) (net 6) (status 30))
 (segment (start 142.111 116.0254) (end 142.111 110.139) (width 0.2032) (layer F.Cu) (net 6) (status 10))
 (segment (start 142.111 110.139) (end 142.35 109.9) (width 0.2032) (layer F.Cu) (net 6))
 (segment (start 142.35 109.9) (end 142.619 110.169) (width 0.2032) (layer F.Cu) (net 6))
 (segment (start 142.619 110.169) (end 142.619 116.0254) (width 0.2032) (layer F.Cu) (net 6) (status 20))
 (segment (start 146.15 110) (end 146.4671 110.3171) (width 0.2032) (layer F.Cu) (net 4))
 (segment (start 146.4671 110.3171) (end 146.4671 116.2794) (width 0.2032) (layer F.Cu) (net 4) (status 20))
 (segment (start 146.15 110) (end 145.8829 110.2671) (width 0.2032) (layer F.Cu) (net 4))
 (segment (start 145.8829 110.2671) (end 145.8829 116.2794) (width 0.2032) (layer F.Cu) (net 4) (status 20))
 (segment (start 145.075 106.975) (end 145.075 107.554) (width 0.254) (layer F.Cu) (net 4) (status 10))
 (segment (start 145.075 107.554) (end 146.15 108.629) (width 0.254) (layer F.Cu) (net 4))
 (segment (start 146.15 108.629) (end 146.15 110) (width 0.254) (layer F.Cu) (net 4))
 (segment (start 140.925 106.975) (end 145.075 106.975) (width 0.254) (layer F.Cu) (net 4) (status 30))
 (segment (start 145.54 97.8) (end 145.54 103.937078) (width 0.254) (layer F.Cu) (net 4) (status 10))
 (segment (start 145.54 103.937078) (end 145.879401 104.276479) (width 0.254) (layer F.Cu) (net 4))
 (segment (start 145.879401 104.276479) (end 145.879401 105.591599) (width 0.254) (layer F.Cu) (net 4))
 (segment (start 145.879401 105.591599) (end 145.075 106.396) (width 0.254) (layer F.Cu) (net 4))
 (segment (start 145.075 106.396) (end 145.075 106.975) (width 0.254) (layer F.Cu) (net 4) (status 20))
 (segment (start 145.075 106.975) (end 145.275 106.975) (width 0.4572) (layer F.Cu) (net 4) (status 30))
 (segment (start 145.25 109.05) (end 145.25 109.481052) (width 0.254) (layer F.Cu) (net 7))
 (via (at 145.25 109.05) (size 0.6096) (drill 0.3) (layers F.Cu B.Cu) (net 7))
 (segment (start 144.9 109.831052) (end 144.9 109.9) (width 0.254) (layer F.Cu) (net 7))
 (segment (start 145.25 109.481052) (end 144.9 109.831052) (width 0.254) (layer F.Cu) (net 7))
 (segment (start 144.9 109.9) (end 145.159 110.159) (width 0.2032) (layer F.Cu) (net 7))
 (segment (start 145.159 110.159) (end 145.159 116.0254) (width 0.2032) (layer F.Cu) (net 7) (status 20))
 (segment (start 144.651 110.149) (end 144.9 109.9) (width 0.2032) (layer F.Cu) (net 7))
 (segment (start 144.651 116.0254) (end 144.651 110.149) (width 0.2032) (layer F.Cu) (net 7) (status 10))
 (segment (start 143 101.8) (end 145.25 104.05) (width 0.254) (layer B.Cu) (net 7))
 (segment (start 143 97.8) (end 143 101.8) (width 0.254) (layer B.Cu) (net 7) (status 10))
 (segment (start 145.25 104.05) (end 145.25 109.05) (width 0.254) (layer B.Cu) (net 7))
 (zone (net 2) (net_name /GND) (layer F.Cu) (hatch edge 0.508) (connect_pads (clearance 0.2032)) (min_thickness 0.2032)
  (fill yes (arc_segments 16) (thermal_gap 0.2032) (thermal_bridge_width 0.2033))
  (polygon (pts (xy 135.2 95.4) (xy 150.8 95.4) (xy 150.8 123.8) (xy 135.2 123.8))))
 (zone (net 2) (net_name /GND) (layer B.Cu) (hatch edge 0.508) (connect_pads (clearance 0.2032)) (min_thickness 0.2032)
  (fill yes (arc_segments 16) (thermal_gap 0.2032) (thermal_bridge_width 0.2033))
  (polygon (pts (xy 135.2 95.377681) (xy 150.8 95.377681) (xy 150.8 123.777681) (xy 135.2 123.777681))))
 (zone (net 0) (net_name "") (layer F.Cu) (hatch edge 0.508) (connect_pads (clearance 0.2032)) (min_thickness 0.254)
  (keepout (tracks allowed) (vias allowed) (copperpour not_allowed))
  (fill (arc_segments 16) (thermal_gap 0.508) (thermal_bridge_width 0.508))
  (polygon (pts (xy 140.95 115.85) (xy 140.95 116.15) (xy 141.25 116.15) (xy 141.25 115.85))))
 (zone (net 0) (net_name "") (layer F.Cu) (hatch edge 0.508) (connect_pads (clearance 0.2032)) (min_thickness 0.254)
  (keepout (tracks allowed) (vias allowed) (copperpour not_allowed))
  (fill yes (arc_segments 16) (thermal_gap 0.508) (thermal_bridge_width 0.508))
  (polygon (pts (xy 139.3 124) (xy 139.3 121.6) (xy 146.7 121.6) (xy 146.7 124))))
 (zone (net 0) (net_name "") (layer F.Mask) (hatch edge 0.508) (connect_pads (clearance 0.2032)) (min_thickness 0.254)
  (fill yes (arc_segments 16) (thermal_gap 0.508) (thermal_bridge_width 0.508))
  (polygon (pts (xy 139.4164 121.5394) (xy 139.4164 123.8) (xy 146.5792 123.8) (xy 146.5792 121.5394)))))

